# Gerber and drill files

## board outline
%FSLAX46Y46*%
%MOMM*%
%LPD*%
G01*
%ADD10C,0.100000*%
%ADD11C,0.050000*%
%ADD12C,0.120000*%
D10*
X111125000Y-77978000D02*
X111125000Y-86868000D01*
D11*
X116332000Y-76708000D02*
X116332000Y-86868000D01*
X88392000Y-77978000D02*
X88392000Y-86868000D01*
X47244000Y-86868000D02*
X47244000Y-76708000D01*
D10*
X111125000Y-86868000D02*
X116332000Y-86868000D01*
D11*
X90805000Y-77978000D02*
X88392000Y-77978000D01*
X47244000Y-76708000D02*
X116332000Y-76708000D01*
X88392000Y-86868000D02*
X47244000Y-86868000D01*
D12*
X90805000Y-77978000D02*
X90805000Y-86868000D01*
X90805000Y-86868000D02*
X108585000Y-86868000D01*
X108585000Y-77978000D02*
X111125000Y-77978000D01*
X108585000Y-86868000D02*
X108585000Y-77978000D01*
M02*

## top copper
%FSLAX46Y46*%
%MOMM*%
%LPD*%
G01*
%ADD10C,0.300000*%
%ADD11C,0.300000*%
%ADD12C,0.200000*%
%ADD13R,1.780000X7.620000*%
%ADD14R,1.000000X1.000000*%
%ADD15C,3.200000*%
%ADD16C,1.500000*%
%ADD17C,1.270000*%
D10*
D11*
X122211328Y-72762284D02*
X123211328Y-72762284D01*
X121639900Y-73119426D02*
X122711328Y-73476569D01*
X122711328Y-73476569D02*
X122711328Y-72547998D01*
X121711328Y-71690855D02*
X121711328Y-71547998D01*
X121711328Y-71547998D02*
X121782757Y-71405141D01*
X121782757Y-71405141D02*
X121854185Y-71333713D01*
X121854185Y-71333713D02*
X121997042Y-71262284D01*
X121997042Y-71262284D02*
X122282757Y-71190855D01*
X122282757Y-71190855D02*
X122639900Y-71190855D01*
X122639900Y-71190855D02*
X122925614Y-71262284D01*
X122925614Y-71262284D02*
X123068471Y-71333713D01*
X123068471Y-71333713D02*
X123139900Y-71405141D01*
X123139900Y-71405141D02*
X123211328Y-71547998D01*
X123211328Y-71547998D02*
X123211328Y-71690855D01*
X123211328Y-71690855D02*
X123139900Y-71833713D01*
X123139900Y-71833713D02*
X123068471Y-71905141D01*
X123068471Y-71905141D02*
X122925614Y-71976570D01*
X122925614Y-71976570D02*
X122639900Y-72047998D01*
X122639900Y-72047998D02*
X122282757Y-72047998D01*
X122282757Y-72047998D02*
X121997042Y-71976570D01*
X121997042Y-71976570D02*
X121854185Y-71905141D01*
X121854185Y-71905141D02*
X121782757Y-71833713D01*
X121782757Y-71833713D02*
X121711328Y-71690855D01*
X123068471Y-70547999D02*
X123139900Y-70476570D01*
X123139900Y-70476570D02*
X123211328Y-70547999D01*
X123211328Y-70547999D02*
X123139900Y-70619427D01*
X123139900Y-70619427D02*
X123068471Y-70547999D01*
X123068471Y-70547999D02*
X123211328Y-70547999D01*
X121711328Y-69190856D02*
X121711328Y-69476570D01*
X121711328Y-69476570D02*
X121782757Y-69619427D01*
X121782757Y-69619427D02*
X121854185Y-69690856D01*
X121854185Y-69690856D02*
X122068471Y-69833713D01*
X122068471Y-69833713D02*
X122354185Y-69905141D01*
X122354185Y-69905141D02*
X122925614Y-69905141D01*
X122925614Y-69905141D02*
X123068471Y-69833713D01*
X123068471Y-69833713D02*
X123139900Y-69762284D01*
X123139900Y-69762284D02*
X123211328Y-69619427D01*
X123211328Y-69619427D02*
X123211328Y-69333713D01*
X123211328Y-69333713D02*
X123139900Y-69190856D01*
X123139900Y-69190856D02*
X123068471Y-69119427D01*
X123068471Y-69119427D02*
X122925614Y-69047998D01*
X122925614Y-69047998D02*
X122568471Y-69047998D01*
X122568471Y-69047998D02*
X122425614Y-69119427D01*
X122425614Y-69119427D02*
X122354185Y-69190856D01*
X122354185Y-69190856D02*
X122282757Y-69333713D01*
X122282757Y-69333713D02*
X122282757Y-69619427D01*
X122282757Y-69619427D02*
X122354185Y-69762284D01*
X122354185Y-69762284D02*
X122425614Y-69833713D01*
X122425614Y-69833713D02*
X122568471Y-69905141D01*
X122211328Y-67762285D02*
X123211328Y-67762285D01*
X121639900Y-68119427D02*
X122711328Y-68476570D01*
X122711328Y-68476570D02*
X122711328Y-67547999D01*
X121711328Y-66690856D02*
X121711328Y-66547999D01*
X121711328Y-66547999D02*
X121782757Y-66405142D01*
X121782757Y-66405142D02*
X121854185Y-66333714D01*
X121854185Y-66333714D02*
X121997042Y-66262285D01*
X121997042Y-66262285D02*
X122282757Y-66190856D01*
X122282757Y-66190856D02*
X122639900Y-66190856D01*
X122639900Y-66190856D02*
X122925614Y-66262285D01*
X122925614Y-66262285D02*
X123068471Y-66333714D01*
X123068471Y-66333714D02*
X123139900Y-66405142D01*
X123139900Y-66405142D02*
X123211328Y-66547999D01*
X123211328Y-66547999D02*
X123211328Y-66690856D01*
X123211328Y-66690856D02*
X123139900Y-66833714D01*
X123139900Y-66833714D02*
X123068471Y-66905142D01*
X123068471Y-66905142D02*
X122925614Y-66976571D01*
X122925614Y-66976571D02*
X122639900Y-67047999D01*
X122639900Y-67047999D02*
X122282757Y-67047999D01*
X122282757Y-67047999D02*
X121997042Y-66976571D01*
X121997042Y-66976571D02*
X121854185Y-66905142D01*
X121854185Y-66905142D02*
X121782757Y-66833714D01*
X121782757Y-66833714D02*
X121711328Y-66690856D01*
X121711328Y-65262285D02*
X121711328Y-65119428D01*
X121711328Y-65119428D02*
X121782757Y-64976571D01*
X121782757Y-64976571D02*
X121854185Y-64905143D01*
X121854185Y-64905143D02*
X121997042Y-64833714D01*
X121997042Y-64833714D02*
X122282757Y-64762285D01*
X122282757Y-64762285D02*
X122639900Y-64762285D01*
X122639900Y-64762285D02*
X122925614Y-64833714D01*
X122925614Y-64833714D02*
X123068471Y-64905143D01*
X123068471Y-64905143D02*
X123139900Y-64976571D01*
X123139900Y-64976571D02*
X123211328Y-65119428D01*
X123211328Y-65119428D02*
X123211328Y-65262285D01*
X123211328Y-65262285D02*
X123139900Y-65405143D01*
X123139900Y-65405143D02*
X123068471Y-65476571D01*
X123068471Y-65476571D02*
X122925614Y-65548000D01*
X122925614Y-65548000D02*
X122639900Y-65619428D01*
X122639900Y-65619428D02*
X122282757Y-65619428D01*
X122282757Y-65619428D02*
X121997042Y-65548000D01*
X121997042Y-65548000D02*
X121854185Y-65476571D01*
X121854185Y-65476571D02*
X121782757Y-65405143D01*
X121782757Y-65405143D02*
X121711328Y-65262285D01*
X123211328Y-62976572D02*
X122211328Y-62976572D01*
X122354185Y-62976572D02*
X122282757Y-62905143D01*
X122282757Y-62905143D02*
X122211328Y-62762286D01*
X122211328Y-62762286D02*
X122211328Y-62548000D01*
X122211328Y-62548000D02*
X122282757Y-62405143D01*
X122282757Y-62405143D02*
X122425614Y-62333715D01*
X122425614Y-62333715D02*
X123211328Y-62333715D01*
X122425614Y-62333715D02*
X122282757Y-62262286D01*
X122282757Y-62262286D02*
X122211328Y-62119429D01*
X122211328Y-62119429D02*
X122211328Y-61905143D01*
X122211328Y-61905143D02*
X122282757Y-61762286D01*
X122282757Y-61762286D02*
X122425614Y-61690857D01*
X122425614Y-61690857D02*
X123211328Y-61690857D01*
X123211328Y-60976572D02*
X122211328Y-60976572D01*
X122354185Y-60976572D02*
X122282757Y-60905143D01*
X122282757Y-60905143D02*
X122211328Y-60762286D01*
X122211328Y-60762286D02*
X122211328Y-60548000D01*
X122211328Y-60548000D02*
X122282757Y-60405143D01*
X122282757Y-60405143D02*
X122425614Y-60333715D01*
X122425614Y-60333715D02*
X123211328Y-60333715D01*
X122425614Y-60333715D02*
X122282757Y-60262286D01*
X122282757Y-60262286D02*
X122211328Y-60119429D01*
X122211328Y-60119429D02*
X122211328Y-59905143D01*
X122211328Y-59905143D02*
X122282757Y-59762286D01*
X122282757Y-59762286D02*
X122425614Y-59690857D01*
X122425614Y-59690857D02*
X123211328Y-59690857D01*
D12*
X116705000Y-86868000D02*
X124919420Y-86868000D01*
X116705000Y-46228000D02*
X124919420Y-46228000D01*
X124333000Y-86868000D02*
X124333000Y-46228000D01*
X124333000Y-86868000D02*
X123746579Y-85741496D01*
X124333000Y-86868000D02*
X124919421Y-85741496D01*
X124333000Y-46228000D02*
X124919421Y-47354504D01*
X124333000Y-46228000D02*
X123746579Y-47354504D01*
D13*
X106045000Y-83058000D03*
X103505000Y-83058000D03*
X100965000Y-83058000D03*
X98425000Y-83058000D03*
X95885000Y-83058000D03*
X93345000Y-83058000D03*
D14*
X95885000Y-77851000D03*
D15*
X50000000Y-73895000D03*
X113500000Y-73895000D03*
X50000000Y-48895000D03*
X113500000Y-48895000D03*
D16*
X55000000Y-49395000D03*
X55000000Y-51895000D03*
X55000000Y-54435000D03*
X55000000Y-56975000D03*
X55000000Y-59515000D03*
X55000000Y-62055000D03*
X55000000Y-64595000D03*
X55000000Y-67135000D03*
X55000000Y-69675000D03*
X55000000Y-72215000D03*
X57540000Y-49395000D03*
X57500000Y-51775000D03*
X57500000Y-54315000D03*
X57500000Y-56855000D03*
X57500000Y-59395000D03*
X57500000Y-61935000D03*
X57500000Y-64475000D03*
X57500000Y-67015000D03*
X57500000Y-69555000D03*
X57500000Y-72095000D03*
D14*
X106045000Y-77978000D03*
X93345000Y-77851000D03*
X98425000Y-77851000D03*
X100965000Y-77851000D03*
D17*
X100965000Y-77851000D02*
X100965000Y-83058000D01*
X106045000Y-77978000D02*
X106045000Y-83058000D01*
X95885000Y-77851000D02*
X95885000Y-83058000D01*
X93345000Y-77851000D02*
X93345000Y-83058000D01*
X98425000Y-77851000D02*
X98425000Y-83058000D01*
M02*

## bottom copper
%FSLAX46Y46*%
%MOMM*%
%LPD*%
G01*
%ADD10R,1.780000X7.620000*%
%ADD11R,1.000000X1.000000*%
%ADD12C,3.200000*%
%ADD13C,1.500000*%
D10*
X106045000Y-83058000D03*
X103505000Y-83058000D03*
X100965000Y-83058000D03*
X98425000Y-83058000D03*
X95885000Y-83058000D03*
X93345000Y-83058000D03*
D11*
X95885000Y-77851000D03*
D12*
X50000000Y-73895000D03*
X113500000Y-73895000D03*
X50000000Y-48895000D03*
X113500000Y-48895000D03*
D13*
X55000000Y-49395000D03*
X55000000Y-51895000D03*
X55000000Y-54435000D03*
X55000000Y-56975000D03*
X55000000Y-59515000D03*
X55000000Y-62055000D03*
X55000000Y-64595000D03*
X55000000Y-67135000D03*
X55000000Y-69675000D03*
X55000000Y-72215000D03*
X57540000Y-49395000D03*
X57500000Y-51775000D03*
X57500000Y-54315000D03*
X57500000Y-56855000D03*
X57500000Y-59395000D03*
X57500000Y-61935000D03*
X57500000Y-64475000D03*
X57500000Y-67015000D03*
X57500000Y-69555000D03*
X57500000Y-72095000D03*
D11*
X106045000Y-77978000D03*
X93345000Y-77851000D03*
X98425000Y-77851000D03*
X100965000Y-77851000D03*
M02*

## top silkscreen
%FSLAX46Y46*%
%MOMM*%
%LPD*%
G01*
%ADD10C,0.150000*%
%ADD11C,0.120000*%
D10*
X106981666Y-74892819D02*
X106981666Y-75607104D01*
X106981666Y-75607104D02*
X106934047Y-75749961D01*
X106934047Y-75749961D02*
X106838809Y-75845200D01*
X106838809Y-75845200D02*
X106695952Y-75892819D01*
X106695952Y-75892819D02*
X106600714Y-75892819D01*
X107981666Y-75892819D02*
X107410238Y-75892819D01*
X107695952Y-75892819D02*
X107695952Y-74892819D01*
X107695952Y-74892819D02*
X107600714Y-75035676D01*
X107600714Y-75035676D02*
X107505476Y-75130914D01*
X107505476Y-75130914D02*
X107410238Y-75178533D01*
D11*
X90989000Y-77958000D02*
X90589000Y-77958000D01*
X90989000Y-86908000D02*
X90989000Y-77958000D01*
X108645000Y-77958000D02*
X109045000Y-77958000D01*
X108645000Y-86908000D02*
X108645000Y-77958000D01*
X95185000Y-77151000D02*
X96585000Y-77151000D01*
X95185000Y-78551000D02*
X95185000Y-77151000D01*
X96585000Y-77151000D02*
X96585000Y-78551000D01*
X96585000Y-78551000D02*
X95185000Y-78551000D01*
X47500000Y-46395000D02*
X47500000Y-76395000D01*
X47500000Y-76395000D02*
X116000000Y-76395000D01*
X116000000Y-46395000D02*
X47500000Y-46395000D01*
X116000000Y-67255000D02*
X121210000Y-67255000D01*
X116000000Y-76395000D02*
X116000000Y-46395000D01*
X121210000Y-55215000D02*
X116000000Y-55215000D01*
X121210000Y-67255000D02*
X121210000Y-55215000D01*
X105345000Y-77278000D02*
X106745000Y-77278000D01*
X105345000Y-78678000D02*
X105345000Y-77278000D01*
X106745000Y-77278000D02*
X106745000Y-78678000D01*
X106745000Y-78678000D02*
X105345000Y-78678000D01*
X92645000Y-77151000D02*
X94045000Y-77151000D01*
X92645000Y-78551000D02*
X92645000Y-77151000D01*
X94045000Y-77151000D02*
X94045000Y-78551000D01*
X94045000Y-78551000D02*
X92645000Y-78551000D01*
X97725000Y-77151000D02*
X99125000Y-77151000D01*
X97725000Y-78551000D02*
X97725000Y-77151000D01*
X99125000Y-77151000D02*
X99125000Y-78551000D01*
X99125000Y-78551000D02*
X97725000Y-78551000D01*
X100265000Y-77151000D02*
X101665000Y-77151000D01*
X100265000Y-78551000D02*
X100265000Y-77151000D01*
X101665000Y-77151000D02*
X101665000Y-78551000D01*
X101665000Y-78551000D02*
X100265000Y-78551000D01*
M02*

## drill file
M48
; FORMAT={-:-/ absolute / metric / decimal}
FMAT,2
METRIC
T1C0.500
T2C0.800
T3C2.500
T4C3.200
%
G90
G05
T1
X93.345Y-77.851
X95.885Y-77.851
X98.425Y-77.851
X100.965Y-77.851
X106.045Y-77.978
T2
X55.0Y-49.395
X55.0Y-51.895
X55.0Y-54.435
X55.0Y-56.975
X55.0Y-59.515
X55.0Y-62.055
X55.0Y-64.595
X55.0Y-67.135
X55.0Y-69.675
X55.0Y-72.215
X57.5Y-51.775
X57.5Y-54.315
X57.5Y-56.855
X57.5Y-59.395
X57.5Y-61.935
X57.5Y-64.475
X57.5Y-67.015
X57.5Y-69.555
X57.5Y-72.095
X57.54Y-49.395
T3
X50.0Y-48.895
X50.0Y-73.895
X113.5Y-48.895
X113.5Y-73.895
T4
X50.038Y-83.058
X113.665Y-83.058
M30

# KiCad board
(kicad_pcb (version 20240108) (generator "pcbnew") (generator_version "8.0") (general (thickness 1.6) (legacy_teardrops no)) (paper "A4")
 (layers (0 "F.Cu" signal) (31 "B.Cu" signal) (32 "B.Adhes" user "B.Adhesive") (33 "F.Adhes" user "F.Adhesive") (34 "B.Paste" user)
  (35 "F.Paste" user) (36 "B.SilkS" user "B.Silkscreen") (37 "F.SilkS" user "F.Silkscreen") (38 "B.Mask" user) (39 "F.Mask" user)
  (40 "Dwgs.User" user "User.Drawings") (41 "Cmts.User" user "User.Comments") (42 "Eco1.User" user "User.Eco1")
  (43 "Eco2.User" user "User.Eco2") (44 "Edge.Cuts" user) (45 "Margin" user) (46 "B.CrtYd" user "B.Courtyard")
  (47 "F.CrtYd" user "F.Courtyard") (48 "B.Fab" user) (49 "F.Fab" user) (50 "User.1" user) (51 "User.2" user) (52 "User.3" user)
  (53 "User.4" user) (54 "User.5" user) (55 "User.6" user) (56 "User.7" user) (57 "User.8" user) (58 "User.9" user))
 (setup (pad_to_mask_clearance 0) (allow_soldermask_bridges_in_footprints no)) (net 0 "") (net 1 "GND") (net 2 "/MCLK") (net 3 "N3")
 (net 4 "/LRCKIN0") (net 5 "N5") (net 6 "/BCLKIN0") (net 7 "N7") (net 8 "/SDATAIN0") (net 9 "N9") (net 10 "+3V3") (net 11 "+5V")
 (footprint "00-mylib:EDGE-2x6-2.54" (layer "F.Cu") (at 99.695 83.058)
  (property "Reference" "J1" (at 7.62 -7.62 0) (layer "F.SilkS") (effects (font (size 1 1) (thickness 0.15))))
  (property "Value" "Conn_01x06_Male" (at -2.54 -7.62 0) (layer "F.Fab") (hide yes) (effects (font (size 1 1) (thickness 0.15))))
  (fp_line (start -8.706 -5.1) (end -9.106 -5.1) (stroke (width 0.12) (type solid)) (layer "F.SilkS"))
  (fp_line (start -8.706 3.85) (end -8.706 -5.1) (stroke (width 0.12) (type solid)) (layer "F.SilkS"))
  (fp_line (start 8.95 -5.1) (end 9.35 -5.1) (stroke (width 0.12) (type solid)) (layer "F.SilkS"))
  (fp_line (start 8.95 3.85) (end 8.95 -5.1) (stroke (width 0.12) (type solid)) (layer "F.SilkS"))
  (fp_line (start -8.89 -5.08) (end -8.89 3.81) (stroke (width 0.12) (type default)) (layer "Edge.Cuts"))
  (fp_line (start -8.89 3.81) (end 8.89 3.81) (stroke (width 0.12) (type default)) (layer "Edge.Cuts"))
  (fp_line (start 8.89 -5.08) (end 11.43 -5.08) (stroke (width 0.12) (type default)) (layer "Edge.Cuts"))
  (fp_line (start 8.89 3.81) (end 8.89 -5.08) (stroke (width 0.12) (type default)) (layer "Edge.Cuts"))
  (pad "1" connect rect (at 6.35 0) (size 1.78 7.62) (layers "F.Cu" "F.Mask") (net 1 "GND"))
  (pad "2" connect rect (at 6.35 0) (size 1.78 7.62) (layers "B.Cu" "B.Mask") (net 1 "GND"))
  (pad "3" connect rect (at 3.81 0) (size 1.78 7.62) (layers "F.Cu" "F.Mask") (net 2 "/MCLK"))
  (pad "4" connect rect (at 3.81 0) (size 1.78 7.62) (layers "B.Cu" "B.Mask") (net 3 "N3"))
  (pad "5" connect rect (at 1.27 0) (size 1.78 7.62) (layers "F.Cu" "F.Mask") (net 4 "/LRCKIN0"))
  (pad "6" connect rect (at 1.27 0) (size 1.78 7.62) (layers "B.Cu" "B.Mask") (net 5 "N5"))
  (pad "7" connect rect (at -1.27 0) (size 1.78 7.62) (layers "F.Cu" "F.Mask") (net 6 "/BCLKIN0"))
  (pad "8" connect rect (at -1.27 0) (size 1.78 7.62) (layers "B.Cu" "B.Mask") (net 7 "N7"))
  (pad "9" connect rect (at -3.81 0) (size 1.78 7.62) (layers "F.Cu" "F.Mask") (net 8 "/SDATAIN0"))
  (pad "10" connect rect (at -3.81 0) (size 1.78 7.62) (layers "B.Cu" "B.Mask") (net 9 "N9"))
  (pad "11" connect rect (at -6.35 0) (size 1.78 7.62) (layers "F.Cu" "F.Mask") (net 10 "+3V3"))
  (pad "12" connect rect (at -6.35 0) (size 1.78 7.62) (layers "B.Cu" "B.Mask") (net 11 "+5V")))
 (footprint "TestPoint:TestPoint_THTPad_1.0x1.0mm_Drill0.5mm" (layer "F.Cu") (at 95.885 77.851)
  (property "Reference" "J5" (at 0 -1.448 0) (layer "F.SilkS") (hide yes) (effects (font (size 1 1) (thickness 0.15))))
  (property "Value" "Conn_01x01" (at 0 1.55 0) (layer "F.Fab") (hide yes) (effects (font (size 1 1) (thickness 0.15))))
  (fp_line (start -0.7 -0.7) (end 0.7 -0.7) (stroke (width 0.12) (type solid)) (layer "F.SilkS"))
  (fp_line (start -0.7 0.7) (end -0.7 -0.7) (stroke (width 0.12) (type solid)) (layer "F.SilkS"))
  (fp_line (start 0.7 -0.7) (end 0.7 0.7) (stroke (width 0.12) (type solid)) (layer "F.SilkS"))
  (fp_line (start 0.7 0.7) (end -0.7 0.7) (stroke (width 0.12) (type solid)) (layer "F.SilkS"))
  (pad "1" thru_hole rect (at 0 0) (size 1 1) (drill 0.5) (layers "*.Cu" "*.Mask") (remove_unused_layers no) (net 8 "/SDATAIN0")))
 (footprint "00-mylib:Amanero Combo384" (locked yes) (layer "F.Cu") (at 116 76.395 90)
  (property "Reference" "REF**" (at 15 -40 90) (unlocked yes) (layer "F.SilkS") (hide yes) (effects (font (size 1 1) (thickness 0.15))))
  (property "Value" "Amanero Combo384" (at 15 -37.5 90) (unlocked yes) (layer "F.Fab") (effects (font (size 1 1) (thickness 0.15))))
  (fp_line (start 30 -68.5) (end 0 -68.5) (stroke (width 0.12) (type solid)) (layer "F.SilkS"))
  (fp_line (start 0 -68.5) (end 0 0) (stroke (width 0.12) (type solid)) (layer "F.SilkS"))
  (fp_line (start 30 0) (end 30 -68.5) (stroke (width 0.12) (type solid)) (layer "F.SilkS"))
  (fp_line (start 9.14 0) (end 9.14 5.21) (stroke (width 0.12) (type solid)) (layer "F.SilkS"))
  (fp_line (start 0 0) (end 30 0) (stroke (width 0.12) (type solid)) (layer "F.SilkS"))
  (fp_line (start 21.18 5.21) (end 21.18 0) (stroke (width 0.12) (type solid)) (layer "F.SilkS"))
  (fp_line (start 9.14 5.21) (end 21.18 5.21) (stroke (width 0.12) (type solid)) (layer "F.SilkS"))
  (pad "" np_thru_hole circle (at 2.5 -66 90) (size 3.2 3.2) (drill 2.5) (layers "F&B.Cu" "*.Mask"))
  (pad "" np_thru_hole circle (at 2.5 -2.5 90) (size 3.2 3.2) (drill 2.5) (layers "F&B.Cu" "*.Mask"))
  (pad "" np_thru_hole circle (at 27.5 -66 90) (size 3.2 3.2) (drill 2.5) (layers "F&B.Cu" "*.Mask"))
  (pad "" np_thru_hole circle (at 27.5 -2.5 90) (size 3.2 3.2) (drill 2.5) (layers "F&B.Cu" "*.Mask"))
  (pad "1" thru_hole circle (at 27 -61 90) (size 1.5 1.5) (drill 0.8) (layers "*.Cu" "*.Mask") (remove_unused_layers no))
  (pad "2" thru_hole circle (at 24.5 -61 270) (size 1.5 1.5) (drill 0.8) (layers "*.Cu" "*.Mask") (remove_unused_layers no))
  (pad "3" thru_hole circle (at 21.96 -61 270) (size 1.5 1.5) (drill 0.8) (layers "*.Cu" "*.Mask") (remove_unused_layers no))
  (pad "4" thru_hole circle (at 19.42 -61 270) (size 1.5 1.5) (drill 0.8) (layers "*.Cu" "*.Mask") (remove_unused_layers no))
  (pad "5" thru_hole circle (at 16.88 -61 270) (size 1.5 1.5) (drill 0.8) (layers "*.Cu" "*.Mask") (remove_unused_layers no))
  (pad "6" thru_hole circle (at 14.34 -61 270) (size 1.5 1.5) (drill 0.8) (layers "*.Cu" "*.Mask") (remove_unused_layers no))
  (pad "7" thru_hole circle (at 11.8 -61 270) (size 1.5 1.5) (drill 0.8) (layers "*.Cu" "*.Mask") (remove_unused_layers no))
  (pad "8" thru_hole circle (at 9.26 -61 270) (size 1.5 1.5) (drill 0.8) (layers "*.Cu" "*.Mask") (remove_unused_layers no))
  (pad "9" thru_hole circle (at 6.72 -61 270) (size 1.5 1.5) (drill 0.8) (layers "*.Cu" "*.Mask") (remove_unused_layers no))
  (pad "10" thru_hole circle (at 4.18 -61 270) (size 1.5 1.5) (drill 0.8) (layers "*.Cu" "*.Mask") (remove_unused_layers no))
  (pad "11" thru_hole circle (at 27 -58.46 90) (size 1.5 1.5) (drill 0.8) (layers "*.Cu" "*.Mask") (remove_unused_layers no))
  (pad "12" thru_hole circle (at 24.62 -58.5 270) (size 1.5 1.5) (drill 0.8) (layers "*.Cu" "*.Mask") (remove_unused_layers no))
  (pad "13" thru_hole circle (at 22.08 -58.5 270) (size 1.5 1.5) (drill 0.8) (layers "*.Cu" "*.Mask") (remove_unused_layers no))
  (pad "14" thru_hole circle (at 19.54 -58.5 270) (size 1.5 1.5) (drill 0.8) (layers "*.Cu" "*.Mask") (remove_unused_layers no))
  (pad "15" thru_hole circle (at 17 -58.5 270) (size 1.5 1.5) (drill 0.8) (layers "*.Cu" "*.Mask") (remove_unused_layers no))
  (pad "16" thru_hole circle (at 14.46 -58.5 270) (size 1.5 1.5) (drill 0.8) (layers "*.Cu" "*.Mask") (remove_unused_layers no))
  (pad "17" thru_hole circle (at 11.92 -58.5 270) (size 1.5 1.5) (drill 0.8) (layers "*.Cu" "*.Mask") (remove_unused_layers no))
  (pad "18" thru_hole circle (at 9.38 -58.5 270) (size 1.5 1.5) (drill 0.8) (layers "*.Cu" "*.Mask") (remove_unused_layers no))
  (pad "19" thru_hole circle (at 6.84 -58.5 270) (size 1.5 1.5) (drill 0.8) (layers "*.Cu" "*.Mask") (remove_unused_layers no))
  (pad "20" thru_hole circle (at 4.3 -58.5 270) (size 1.5 1.5) (drill 0.8) (layers "*.Cu" "*.Mask") (remove_unused_layers no)))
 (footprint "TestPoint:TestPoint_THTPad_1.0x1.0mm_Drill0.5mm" (layer "F.Cu") (at 106.045 77.978)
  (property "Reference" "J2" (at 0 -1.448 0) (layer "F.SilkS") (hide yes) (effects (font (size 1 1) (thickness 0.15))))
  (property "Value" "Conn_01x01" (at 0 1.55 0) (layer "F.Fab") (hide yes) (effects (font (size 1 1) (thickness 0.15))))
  (fp_line (start -0.7 -0.7) (end 0.7 -0.7) (stroke (width 0.12) (type solid)) (layer "F.SilkS"))
  (fp_line (start -0.7 0.7) (end -0.7 -0.7) (stroke (width 0.12) (type solid)) (layer "F.SilkS"))
  (fp_line (start 0.7 -0.7) (end 0.7 0.7) (stroke (width 0.12) (type solid)) (layer "F.SilkS"))
  (fp_line (start 0.7 0.7) (end -0.7 0.7) (stroke (width 0.12) (type solid)) (layer "F.SilkS"))
  (pad "1" thru_hole rect (at 0 0) (size 1 1) (drill 0.5) (layers "*.Cu" "*.Mask") (remove_unused_layers no) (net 1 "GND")))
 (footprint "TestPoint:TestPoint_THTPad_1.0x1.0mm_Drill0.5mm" (layer "F.Cu") (at 93.345 77.851)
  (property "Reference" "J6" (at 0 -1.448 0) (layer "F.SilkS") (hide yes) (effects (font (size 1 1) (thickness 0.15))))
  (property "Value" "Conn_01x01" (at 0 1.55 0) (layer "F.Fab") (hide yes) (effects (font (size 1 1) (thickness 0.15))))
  (fp_line (start -0.7 -0.7) (end 0.7 -0.7) (stroke (width 0.12) (type solid)) (layer "F.SilkS"))
  (fp_line (start -0.7 0.7) (end -0.7 -0.7) (stroke (width 0.12) (type solid)) (layer "F.SilkS"))
  (fp_line (start 0.7 -0.7) (end 0.7 0.7) (stroke (width 0.12) (type solid)) (layer "F.SilkS"))
  (fp_line (start 0.7 0.7) (end -0.7 0.7) (stroke (width 0.12) (type solid)) (layer "F.SilkS"))
  (pad "1" thru_hole rect (at 0 0) (size 1 1) (drill 0.5) (layers "*.Cu" "*.Mask") (remove_unused_layers no) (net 10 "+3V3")))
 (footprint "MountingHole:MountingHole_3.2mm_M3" (layer "F.Cu") (at 113.665 83.058)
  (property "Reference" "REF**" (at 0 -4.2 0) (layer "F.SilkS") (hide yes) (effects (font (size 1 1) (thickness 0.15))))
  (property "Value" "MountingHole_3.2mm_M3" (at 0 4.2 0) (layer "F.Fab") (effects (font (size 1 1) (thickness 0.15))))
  (pad "" np_thru_hole circle (at 0 0) (size 3.2 3.2) (drill 3.2) (layers "F&B.Cu" "*.Mask")))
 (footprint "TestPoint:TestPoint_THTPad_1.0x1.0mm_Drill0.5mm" (layer "F.Cu") (at 98.425 77.851)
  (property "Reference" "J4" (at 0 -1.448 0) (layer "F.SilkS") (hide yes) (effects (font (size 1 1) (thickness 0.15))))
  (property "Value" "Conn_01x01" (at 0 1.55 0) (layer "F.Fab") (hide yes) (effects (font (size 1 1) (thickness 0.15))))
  (fp_line (start -0.7 -0.7) (end 0.7 -0.7) (stroke (width 0.12) (type solid)) (layer "F.SilkS"))
  (fp_line (start -0.7 0.7) (end -0.7 -0.7) (stroke (width 0.12) (type solid)) (layer "F.SilkS"))
  (fp_line (start 0.7 -0.7) (end 0.7 0.7) (stroke (width 0.12) (type solid)) (layer "F.SilkS"))
  (fp_line (start 0.7 0.7) (end -0.7 0.7) (stroke (width 0.12) (type solid)) (layer "F.SilkS"))
  (pad "1" thru_hole rect (at 0 0) (size 1 1) (drill 0.5) (layers "*.Cu" "*.Mask") (remove_unused_layers no) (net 6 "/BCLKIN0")))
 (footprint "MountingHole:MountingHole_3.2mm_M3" (layer "F.Cu") (at 50.038 83.058)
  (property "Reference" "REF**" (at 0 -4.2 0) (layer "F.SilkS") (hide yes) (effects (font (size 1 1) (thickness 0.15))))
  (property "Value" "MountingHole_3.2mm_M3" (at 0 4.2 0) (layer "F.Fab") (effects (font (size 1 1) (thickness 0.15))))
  (pad "" np_thru_hole circle (at 0 0) (size 3.2 3.2) (drill 3.2) (layers "F&B.Cu" "*.Mask")))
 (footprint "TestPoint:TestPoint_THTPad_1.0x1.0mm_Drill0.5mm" (layer "F.Cu") (at 100.965 77.851)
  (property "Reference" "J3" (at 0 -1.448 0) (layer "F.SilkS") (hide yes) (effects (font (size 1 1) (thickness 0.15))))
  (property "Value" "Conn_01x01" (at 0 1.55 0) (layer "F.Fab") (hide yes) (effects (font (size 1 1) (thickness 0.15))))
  (fp_line (start -0.7 -0.7) (end 0.7 -0.7) (stroke (width 0.12) (type solid)) (layer "F.SilkS"))
  (fp_line (start -0.7 0.7) (end -0.7 -0.7) (stroke (width 0.12) (type solid)) (layer "F.SilkS"))
  (fp_line (start 0.7 -0.7) (end 0.7 0.7) (stroke (width 0.12) (type solid)) (layer "F.SilkS"))
  (fp_line (start 0.7 0.7) (end -0.7 0.7) (stroke (width 0.12) (type solid)) (layer "F.SilkS"))
  (pad "1" thru_hole rect (at 0 0) (size 1 1) (drill 0.5) (layers "*.Cu" "*.Mask") (remove_unused_layers no) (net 4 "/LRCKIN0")))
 (gr_line (start 111.125 77.978) (end 111.125 86.868) (stroke (width 0.1) (type default)) (layer "Edge.Cuts"))
 (gr_line (start 116.332 76.708) (end 116.332 86.868) (stroke (width 0.05) (type default)) (layer "Edge.Cuts"))
 (gr_line (start 88.392 77.978) (end 88.392 86.868) (stroke (width 0.05) (type default)) (layer "Edge.Cuts"))
 (gr_line (start 47.244 86.868) (end 47.244 76.708) (stroke (width 0.05) (type default)) (layer "Edge.Cuts"))
 (gr_line (start 111.125 86.868) (end 116.332 86.868) (stroke (width 0.1) (type default)) (layer "Edge.Cuts"))
 (gr_line (start 90.805 77.978) (end 88.392 77.978) (stroke (width 0.05) (type default)) (layer "Edge.Cuts"))
 (gr_line (start 47.244 76.708) (end 116.332 76.708) (stroke (width 0.05) (type default)) (layer "Edge.Cuts"))
 (gr_line (start 88.392 86.868) (end 47.244 86.868) (stroke (width 0.05) (type default)) (layer "Edge.Cuts"))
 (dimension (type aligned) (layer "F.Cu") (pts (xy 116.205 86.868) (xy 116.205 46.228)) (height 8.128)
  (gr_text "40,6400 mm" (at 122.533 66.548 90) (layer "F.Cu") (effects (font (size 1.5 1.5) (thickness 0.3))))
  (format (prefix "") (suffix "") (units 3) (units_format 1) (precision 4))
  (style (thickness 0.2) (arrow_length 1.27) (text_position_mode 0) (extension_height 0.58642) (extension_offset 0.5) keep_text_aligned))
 (segment (start 100.965 77.851) (end 100.965 83.058) (width 1.27) (layer "F.Cu") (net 4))
 (segment (start 106.045 77.978) (end 106.045 83.058) (width 1.27) (layer "F.Cu") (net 1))
 (segment (start 95.885 77.851) (end 95.885 83.058) (width 1.27) (layer "F.Cu") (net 8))
 (segment (start 93.345 77.851) (end 93.345 83.058) (width 1.27) (layer "F.Cu") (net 10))
 (segment (start 98.425 77.851) (end 98.425 83.058) (width 1.27) (layer "F.Cu") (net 6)))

